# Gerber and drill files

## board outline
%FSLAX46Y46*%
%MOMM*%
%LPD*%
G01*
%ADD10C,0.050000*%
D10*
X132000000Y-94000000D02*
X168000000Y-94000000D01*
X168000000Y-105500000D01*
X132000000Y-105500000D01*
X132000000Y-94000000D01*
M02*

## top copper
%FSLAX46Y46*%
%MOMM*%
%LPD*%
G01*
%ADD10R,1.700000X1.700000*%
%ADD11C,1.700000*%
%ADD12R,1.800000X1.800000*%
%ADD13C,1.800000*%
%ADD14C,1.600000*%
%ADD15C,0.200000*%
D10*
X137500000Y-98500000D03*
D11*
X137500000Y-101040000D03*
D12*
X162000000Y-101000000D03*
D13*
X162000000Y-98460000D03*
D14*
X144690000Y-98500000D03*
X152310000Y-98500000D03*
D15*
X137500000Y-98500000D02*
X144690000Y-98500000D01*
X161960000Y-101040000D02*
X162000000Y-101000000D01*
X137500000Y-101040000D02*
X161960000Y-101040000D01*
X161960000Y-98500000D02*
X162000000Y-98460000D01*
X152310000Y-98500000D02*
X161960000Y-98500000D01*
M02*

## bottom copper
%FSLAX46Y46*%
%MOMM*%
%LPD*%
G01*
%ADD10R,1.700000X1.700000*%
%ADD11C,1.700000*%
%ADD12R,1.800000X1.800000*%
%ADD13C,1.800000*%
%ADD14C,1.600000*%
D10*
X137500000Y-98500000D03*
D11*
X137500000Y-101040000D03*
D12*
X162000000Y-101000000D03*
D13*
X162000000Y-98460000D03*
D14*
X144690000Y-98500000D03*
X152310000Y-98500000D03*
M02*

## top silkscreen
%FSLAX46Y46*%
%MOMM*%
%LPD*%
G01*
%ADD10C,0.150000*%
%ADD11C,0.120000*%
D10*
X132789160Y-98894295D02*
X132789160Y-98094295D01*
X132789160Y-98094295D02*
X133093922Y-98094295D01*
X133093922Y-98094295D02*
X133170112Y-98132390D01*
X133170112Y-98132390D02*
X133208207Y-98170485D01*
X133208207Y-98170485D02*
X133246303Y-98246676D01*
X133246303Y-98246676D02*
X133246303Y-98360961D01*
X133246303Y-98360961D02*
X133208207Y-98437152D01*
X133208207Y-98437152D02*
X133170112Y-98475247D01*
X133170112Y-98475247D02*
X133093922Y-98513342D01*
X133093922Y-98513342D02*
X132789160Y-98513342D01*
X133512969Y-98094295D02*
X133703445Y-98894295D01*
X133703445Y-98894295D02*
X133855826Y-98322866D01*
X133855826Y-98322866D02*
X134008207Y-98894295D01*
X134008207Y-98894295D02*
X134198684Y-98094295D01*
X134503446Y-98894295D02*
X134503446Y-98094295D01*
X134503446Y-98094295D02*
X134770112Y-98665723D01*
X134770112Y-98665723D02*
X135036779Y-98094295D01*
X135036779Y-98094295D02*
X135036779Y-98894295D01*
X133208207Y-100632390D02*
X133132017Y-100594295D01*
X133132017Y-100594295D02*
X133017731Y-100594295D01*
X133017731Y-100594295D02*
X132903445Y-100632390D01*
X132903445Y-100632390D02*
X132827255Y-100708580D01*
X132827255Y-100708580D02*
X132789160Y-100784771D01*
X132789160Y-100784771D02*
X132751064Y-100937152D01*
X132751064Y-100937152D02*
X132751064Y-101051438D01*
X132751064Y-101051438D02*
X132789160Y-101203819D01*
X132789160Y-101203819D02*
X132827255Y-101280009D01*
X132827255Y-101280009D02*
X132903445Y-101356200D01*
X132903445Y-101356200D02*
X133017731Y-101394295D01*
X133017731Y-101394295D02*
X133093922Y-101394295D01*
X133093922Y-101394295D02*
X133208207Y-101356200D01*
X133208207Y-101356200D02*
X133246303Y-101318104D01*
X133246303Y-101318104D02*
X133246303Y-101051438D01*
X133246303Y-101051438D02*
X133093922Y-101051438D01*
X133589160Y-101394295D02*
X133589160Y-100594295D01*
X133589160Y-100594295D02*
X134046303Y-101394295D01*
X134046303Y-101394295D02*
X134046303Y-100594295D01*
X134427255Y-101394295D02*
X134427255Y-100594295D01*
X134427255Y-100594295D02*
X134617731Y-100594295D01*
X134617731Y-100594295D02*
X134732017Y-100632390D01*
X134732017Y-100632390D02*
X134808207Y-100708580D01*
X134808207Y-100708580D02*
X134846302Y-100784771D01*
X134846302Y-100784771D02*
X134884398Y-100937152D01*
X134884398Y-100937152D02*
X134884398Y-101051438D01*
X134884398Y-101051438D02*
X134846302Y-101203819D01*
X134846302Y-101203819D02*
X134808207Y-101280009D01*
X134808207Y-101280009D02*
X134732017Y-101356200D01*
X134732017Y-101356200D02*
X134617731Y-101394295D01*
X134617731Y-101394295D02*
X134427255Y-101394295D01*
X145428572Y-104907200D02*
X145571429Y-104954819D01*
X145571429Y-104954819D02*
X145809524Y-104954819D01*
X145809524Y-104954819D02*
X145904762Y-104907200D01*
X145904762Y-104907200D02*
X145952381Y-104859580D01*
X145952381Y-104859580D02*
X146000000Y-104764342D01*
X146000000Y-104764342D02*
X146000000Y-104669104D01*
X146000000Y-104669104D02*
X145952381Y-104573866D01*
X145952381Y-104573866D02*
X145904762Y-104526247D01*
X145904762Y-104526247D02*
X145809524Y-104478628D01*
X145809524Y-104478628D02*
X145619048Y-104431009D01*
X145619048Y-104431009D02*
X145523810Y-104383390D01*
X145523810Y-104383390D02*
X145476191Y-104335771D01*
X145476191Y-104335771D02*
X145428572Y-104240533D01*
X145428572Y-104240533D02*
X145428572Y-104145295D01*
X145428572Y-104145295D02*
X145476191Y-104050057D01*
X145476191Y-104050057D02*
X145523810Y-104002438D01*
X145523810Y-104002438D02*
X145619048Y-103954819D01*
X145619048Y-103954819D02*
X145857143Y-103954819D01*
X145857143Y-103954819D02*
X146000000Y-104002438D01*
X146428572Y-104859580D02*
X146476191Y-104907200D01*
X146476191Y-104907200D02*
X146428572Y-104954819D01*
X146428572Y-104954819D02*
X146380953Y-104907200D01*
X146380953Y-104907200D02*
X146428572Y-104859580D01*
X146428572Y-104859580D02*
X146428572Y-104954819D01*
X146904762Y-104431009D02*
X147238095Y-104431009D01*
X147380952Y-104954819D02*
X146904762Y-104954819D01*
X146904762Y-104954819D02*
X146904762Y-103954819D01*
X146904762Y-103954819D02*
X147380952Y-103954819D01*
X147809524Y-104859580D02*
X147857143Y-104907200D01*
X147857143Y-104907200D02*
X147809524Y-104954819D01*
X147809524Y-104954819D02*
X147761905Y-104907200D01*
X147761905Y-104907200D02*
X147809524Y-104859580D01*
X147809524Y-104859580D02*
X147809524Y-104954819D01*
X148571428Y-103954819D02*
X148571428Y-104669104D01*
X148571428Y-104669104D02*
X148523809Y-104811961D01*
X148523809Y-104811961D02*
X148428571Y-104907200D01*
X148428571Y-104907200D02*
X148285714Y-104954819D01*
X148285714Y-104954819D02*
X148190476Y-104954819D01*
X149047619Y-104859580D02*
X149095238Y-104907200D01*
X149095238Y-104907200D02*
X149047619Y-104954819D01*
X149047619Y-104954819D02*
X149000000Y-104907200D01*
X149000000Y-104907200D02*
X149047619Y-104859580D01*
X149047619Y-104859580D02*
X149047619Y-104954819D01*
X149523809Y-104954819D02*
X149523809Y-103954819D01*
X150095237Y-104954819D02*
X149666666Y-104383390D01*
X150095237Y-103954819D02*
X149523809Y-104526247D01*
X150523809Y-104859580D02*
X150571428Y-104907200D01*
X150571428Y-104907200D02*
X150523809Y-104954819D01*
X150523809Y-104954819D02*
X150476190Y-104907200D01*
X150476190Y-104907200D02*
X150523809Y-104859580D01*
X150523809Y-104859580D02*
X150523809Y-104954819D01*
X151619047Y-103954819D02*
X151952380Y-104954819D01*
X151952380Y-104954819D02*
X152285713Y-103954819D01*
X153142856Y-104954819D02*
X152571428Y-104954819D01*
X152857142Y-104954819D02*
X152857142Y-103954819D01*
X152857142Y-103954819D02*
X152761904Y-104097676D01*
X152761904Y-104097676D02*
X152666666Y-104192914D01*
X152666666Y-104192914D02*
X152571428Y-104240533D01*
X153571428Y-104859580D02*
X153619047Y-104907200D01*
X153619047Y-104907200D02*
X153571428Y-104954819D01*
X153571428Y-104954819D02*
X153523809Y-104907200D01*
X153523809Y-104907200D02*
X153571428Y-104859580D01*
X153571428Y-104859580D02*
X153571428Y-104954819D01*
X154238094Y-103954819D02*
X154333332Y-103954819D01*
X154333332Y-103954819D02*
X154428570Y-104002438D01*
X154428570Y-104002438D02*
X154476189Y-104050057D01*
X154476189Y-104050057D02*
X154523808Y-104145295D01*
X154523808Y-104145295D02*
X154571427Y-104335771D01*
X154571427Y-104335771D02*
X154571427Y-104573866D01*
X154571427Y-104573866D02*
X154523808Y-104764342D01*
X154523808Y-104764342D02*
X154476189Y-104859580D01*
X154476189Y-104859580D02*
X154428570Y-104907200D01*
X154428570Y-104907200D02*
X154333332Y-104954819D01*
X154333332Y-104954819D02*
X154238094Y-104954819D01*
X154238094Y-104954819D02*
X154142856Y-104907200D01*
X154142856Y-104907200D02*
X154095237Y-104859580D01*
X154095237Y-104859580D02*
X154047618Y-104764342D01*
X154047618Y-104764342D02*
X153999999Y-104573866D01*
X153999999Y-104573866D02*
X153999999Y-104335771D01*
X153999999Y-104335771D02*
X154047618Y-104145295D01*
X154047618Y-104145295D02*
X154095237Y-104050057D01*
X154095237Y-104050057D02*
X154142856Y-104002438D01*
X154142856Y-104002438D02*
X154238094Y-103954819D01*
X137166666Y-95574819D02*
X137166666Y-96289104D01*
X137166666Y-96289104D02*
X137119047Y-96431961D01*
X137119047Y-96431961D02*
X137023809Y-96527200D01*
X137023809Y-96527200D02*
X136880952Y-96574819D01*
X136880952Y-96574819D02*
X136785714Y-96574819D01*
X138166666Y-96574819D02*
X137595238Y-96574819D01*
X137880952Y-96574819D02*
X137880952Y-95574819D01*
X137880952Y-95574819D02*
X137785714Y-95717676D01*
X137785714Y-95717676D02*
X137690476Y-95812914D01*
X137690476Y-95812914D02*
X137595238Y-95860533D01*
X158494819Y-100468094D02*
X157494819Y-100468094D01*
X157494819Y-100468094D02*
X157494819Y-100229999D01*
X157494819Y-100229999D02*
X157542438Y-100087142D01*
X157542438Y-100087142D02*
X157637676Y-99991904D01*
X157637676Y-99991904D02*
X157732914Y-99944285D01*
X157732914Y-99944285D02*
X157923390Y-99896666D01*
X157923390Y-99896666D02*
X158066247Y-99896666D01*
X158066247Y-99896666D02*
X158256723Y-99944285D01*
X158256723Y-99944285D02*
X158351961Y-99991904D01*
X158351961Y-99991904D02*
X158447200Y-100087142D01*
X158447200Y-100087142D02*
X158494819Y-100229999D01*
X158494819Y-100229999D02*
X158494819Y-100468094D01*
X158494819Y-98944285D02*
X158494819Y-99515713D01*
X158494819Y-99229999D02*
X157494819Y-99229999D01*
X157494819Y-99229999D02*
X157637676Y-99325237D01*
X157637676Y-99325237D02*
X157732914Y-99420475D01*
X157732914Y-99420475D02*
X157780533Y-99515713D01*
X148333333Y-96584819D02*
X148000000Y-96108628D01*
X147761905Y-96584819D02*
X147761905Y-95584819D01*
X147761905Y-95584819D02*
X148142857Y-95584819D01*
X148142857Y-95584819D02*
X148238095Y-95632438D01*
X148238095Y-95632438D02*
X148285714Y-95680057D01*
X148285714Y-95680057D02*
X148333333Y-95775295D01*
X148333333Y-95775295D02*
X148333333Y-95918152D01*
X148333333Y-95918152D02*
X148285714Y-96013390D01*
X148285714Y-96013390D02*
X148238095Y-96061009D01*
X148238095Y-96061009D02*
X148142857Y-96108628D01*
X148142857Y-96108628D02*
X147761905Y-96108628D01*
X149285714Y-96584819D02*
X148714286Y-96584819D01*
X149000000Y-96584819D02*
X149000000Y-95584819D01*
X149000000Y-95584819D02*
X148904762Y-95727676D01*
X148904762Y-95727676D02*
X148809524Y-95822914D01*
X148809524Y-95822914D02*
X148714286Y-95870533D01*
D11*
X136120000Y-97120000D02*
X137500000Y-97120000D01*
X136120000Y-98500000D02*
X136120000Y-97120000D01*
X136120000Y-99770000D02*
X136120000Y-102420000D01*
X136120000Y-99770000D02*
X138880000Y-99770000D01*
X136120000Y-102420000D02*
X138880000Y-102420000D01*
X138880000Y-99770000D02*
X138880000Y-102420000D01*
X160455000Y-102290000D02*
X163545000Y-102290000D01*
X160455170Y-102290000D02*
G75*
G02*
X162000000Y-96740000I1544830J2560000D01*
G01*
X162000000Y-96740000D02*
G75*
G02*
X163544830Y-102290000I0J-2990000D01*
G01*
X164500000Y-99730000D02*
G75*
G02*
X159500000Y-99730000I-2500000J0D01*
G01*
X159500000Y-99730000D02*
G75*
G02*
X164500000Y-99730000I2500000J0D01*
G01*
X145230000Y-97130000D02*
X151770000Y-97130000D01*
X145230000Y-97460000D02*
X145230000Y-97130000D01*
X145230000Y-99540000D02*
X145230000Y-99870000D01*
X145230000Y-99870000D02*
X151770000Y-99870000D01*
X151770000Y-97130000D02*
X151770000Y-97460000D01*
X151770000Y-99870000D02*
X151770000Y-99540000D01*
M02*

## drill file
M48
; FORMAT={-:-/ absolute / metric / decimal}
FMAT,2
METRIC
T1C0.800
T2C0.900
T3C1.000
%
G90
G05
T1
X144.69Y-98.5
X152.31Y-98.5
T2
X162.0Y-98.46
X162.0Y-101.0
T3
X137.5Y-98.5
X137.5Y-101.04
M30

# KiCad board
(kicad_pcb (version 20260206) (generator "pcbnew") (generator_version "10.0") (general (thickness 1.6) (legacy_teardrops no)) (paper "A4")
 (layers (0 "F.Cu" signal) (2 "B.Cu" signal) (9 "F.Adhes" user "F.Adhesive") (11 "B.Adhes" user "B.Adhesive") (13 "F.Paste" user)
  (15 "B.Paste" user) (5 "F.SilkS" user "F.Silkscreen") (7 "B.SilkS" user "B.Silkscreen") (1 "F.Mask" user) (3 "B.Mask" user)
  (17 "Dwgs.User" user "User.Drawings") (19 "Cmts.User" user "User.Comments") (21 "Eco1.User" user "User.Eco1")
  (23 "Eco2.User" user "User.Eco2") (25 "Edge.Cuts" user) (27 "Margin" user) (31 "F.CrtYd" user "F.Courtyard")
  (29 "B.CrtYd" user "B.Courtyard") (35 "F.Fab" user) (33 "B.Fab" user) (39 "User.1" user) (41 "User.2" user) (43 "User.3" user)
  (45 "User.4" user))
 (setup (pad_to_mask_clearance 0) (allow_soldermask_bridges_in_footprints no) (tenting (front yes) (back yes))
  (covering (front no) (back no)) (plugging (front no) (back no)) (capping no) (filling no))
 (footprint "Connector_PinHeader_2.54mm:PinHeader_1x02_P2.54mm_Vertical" (layer "F.Cu") (at 137.5 98.5)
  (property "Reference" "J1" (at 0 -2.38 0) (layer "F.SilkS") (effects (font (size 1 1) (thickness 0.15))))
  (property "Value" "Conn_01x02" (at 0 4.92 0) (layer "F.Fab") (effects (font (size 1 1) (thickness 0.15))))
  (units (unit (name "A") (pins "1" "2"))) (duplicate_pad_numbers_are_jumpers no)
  (fp_line (start -1.38 -1.38) (end 0 -1.38) (stroke (width 0.12) (type solid)) (layer "F.SilkS"))
  (fp_line (start -1.38 0) (end -1.38 -1.38) (stroke (width 0.12) (type solid)) (layer "F.SilkS"))
  (fp_line (start -1.38 1.27) (end -1.38 3.92) (stroke (width 0.12) (type solid)) (layer "F.SilkS"))
  (fp_line (start -1.38 1.27) (end 1.38 1.27) (stroke (width 0.12) (type solid)) (layer "F.SilkS"))
  (fp_line (start -1.38 3.92) (end 1.38 3.92) (stroke (width 0.12) (type solid)) (layer "F.SilkS"))
  (fp_line (start 1.38 1.27) (end 1.38 3.92) (stroke (width 0.12) (type solid)) (layer "F.SilkS"))
  (pad "1" thru_hole rect (at 0 0) (size 1.7 1.7) (drill 1) (layers "*.Cu" "*.Mask") (remove_unused_layers no) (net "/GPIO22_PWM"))
  (pad "2" thru_hole circle (at 0 2.54) (size 1.7 1.7) (drill 1) (layers "*.Cu" "*.Mask") (remove_unused_layers no) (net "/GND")))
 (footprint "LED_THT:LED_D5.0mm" (layer "F.Cu") (at 162 101 90)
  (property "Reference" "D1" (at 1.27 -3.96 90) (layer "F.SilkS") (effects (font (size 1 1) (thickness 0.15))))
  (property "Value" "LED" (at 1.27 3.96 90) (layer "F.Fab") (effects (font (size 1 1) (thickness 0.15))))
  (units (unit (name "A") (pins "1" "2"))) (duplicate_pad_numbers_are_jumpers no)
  (fp_line (start -1.29 -1.545) (end -1.29 1.545) (stroke (width 0.12) (type solid)) (layer "F.SilkS"))
  (fp_arc (start -1.29 -1.54483) (mid 2.071779 -2.880495) (end 4.26 0) (stroke (width 0.12) (type solid)) (layer "F.SilkS"))
  (fp_arc (start 4.26 0) (mid 2.071779 2.880495) (end -1.29 1.54483) (stroke (width 0.12) (type solid)) (layer "F.SilkS"))
  (fp_circle (center 1.27 0) (end 3.77 0) (stroke (width 0.12) (type solid)) (fill no) (layer "F.SilkS"))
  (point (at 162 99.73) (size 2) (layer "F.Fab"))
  (pad "1" thru_hole rect (at 0 0 90) (size 1.8 1.8) (drill 0.9) (layers "*.Cu" "*.Mask") (remove_unused_layers no) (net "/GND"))
  (pad "2" thru_hole circle (at 2.54 0 90) (size 1.8 1.8) (drill 0.9) (layers "*.Cu" "*.Mask") (remove_unused_layers no) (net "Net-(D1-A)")))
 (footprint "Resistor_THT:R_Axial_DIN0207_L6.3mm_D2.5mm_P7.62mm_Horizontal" (layer "F.Cu") (at 144.69 98.5)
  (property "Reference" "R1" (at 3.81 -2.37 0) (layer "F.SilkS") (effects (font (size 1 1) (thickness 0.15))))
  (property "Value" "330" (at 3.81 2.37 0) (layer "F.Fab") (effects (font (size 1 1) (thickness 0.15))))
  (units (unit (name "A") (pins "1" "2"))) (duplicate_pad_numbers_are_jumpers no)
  (fp_line (start 0.54 -1.37) (end 7.08 -1.37) (stroke (width 0.12) (type solid)) (layer "F.SilkS"))
  (fp_line (start 0.54 -1.04) (end 0.54 -1.37) (stroke (width 0.12) (type solid)) (layer "F.SilkS"))
  (fp_line (start 0.54 1.04) (end 0.54 1.37) (stroke (width 0.12) (type solid)) (layer "F.SilkS"))
  (fp_line (start 0.54 1.37) (end 7.08 1.37) (stroke (width 0.12) (type solid)) (layer "F.SilkS"))
  (fp_line (start 7.08 -1.37) (end 7.08 -1.04) (stroke (width 0.12) (type solid)) (layer "F.SilkS"))
  (fp_line (start 7.08 1.37) (end 7.08 1.04) (stroke (width 0.12) (type solid)) (layer "F.SilkS"))
  (pad "1" thru_hole circle (at 0 0) (size 1.6 1.6) (drill 0.8) (layers "*.Cu" "*.Mask") (remove_unused_layers no) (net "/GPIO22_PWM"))
  (pad "2" thru_hole circle (at 7.62 0) (size 1.6 1.6) (drill 0.8) (layers "*.Cu" "*.Mask") (remove_unused_layers no) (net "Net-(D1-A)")))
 (gr_rect (start 132 94) (end 168 105.5) (stroke (width 0.05) (type default)) (fill no) (layer "Edge.Cuts"))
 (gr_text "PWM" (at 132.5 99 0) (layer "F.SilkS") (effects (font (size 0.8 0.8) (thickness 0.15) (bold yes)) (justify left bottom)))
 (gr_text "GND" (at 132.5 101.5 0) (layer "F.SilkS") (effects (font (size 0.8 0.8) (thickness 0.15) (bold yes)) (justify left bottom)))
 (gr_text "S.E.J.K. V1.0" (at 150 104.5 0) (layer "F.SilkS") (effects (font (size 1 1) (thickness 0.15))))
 (segment (start 137.5 98.5) (end 144.69 98.5) (width 0.2) (layer "F.Cu") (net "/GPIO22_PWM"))
 (segment (start 161.96 101.04) (end 162 101) (width 0.2) (layer "F.Cu") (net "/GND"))
 (segment (start 137.5 101.04) (end 161.96 101.04) (width 0.2) (layer "F.Cu") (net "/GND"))
 (segment (start 161.96 98.5) (end 162 98.46) (width 0.2) (layer "F.Cu") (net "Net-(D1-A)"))
 (segment (start 152.31 98.5) (end 161.96 98.5) (width 0.2) (layer "F.Cu") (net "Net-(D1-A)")))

